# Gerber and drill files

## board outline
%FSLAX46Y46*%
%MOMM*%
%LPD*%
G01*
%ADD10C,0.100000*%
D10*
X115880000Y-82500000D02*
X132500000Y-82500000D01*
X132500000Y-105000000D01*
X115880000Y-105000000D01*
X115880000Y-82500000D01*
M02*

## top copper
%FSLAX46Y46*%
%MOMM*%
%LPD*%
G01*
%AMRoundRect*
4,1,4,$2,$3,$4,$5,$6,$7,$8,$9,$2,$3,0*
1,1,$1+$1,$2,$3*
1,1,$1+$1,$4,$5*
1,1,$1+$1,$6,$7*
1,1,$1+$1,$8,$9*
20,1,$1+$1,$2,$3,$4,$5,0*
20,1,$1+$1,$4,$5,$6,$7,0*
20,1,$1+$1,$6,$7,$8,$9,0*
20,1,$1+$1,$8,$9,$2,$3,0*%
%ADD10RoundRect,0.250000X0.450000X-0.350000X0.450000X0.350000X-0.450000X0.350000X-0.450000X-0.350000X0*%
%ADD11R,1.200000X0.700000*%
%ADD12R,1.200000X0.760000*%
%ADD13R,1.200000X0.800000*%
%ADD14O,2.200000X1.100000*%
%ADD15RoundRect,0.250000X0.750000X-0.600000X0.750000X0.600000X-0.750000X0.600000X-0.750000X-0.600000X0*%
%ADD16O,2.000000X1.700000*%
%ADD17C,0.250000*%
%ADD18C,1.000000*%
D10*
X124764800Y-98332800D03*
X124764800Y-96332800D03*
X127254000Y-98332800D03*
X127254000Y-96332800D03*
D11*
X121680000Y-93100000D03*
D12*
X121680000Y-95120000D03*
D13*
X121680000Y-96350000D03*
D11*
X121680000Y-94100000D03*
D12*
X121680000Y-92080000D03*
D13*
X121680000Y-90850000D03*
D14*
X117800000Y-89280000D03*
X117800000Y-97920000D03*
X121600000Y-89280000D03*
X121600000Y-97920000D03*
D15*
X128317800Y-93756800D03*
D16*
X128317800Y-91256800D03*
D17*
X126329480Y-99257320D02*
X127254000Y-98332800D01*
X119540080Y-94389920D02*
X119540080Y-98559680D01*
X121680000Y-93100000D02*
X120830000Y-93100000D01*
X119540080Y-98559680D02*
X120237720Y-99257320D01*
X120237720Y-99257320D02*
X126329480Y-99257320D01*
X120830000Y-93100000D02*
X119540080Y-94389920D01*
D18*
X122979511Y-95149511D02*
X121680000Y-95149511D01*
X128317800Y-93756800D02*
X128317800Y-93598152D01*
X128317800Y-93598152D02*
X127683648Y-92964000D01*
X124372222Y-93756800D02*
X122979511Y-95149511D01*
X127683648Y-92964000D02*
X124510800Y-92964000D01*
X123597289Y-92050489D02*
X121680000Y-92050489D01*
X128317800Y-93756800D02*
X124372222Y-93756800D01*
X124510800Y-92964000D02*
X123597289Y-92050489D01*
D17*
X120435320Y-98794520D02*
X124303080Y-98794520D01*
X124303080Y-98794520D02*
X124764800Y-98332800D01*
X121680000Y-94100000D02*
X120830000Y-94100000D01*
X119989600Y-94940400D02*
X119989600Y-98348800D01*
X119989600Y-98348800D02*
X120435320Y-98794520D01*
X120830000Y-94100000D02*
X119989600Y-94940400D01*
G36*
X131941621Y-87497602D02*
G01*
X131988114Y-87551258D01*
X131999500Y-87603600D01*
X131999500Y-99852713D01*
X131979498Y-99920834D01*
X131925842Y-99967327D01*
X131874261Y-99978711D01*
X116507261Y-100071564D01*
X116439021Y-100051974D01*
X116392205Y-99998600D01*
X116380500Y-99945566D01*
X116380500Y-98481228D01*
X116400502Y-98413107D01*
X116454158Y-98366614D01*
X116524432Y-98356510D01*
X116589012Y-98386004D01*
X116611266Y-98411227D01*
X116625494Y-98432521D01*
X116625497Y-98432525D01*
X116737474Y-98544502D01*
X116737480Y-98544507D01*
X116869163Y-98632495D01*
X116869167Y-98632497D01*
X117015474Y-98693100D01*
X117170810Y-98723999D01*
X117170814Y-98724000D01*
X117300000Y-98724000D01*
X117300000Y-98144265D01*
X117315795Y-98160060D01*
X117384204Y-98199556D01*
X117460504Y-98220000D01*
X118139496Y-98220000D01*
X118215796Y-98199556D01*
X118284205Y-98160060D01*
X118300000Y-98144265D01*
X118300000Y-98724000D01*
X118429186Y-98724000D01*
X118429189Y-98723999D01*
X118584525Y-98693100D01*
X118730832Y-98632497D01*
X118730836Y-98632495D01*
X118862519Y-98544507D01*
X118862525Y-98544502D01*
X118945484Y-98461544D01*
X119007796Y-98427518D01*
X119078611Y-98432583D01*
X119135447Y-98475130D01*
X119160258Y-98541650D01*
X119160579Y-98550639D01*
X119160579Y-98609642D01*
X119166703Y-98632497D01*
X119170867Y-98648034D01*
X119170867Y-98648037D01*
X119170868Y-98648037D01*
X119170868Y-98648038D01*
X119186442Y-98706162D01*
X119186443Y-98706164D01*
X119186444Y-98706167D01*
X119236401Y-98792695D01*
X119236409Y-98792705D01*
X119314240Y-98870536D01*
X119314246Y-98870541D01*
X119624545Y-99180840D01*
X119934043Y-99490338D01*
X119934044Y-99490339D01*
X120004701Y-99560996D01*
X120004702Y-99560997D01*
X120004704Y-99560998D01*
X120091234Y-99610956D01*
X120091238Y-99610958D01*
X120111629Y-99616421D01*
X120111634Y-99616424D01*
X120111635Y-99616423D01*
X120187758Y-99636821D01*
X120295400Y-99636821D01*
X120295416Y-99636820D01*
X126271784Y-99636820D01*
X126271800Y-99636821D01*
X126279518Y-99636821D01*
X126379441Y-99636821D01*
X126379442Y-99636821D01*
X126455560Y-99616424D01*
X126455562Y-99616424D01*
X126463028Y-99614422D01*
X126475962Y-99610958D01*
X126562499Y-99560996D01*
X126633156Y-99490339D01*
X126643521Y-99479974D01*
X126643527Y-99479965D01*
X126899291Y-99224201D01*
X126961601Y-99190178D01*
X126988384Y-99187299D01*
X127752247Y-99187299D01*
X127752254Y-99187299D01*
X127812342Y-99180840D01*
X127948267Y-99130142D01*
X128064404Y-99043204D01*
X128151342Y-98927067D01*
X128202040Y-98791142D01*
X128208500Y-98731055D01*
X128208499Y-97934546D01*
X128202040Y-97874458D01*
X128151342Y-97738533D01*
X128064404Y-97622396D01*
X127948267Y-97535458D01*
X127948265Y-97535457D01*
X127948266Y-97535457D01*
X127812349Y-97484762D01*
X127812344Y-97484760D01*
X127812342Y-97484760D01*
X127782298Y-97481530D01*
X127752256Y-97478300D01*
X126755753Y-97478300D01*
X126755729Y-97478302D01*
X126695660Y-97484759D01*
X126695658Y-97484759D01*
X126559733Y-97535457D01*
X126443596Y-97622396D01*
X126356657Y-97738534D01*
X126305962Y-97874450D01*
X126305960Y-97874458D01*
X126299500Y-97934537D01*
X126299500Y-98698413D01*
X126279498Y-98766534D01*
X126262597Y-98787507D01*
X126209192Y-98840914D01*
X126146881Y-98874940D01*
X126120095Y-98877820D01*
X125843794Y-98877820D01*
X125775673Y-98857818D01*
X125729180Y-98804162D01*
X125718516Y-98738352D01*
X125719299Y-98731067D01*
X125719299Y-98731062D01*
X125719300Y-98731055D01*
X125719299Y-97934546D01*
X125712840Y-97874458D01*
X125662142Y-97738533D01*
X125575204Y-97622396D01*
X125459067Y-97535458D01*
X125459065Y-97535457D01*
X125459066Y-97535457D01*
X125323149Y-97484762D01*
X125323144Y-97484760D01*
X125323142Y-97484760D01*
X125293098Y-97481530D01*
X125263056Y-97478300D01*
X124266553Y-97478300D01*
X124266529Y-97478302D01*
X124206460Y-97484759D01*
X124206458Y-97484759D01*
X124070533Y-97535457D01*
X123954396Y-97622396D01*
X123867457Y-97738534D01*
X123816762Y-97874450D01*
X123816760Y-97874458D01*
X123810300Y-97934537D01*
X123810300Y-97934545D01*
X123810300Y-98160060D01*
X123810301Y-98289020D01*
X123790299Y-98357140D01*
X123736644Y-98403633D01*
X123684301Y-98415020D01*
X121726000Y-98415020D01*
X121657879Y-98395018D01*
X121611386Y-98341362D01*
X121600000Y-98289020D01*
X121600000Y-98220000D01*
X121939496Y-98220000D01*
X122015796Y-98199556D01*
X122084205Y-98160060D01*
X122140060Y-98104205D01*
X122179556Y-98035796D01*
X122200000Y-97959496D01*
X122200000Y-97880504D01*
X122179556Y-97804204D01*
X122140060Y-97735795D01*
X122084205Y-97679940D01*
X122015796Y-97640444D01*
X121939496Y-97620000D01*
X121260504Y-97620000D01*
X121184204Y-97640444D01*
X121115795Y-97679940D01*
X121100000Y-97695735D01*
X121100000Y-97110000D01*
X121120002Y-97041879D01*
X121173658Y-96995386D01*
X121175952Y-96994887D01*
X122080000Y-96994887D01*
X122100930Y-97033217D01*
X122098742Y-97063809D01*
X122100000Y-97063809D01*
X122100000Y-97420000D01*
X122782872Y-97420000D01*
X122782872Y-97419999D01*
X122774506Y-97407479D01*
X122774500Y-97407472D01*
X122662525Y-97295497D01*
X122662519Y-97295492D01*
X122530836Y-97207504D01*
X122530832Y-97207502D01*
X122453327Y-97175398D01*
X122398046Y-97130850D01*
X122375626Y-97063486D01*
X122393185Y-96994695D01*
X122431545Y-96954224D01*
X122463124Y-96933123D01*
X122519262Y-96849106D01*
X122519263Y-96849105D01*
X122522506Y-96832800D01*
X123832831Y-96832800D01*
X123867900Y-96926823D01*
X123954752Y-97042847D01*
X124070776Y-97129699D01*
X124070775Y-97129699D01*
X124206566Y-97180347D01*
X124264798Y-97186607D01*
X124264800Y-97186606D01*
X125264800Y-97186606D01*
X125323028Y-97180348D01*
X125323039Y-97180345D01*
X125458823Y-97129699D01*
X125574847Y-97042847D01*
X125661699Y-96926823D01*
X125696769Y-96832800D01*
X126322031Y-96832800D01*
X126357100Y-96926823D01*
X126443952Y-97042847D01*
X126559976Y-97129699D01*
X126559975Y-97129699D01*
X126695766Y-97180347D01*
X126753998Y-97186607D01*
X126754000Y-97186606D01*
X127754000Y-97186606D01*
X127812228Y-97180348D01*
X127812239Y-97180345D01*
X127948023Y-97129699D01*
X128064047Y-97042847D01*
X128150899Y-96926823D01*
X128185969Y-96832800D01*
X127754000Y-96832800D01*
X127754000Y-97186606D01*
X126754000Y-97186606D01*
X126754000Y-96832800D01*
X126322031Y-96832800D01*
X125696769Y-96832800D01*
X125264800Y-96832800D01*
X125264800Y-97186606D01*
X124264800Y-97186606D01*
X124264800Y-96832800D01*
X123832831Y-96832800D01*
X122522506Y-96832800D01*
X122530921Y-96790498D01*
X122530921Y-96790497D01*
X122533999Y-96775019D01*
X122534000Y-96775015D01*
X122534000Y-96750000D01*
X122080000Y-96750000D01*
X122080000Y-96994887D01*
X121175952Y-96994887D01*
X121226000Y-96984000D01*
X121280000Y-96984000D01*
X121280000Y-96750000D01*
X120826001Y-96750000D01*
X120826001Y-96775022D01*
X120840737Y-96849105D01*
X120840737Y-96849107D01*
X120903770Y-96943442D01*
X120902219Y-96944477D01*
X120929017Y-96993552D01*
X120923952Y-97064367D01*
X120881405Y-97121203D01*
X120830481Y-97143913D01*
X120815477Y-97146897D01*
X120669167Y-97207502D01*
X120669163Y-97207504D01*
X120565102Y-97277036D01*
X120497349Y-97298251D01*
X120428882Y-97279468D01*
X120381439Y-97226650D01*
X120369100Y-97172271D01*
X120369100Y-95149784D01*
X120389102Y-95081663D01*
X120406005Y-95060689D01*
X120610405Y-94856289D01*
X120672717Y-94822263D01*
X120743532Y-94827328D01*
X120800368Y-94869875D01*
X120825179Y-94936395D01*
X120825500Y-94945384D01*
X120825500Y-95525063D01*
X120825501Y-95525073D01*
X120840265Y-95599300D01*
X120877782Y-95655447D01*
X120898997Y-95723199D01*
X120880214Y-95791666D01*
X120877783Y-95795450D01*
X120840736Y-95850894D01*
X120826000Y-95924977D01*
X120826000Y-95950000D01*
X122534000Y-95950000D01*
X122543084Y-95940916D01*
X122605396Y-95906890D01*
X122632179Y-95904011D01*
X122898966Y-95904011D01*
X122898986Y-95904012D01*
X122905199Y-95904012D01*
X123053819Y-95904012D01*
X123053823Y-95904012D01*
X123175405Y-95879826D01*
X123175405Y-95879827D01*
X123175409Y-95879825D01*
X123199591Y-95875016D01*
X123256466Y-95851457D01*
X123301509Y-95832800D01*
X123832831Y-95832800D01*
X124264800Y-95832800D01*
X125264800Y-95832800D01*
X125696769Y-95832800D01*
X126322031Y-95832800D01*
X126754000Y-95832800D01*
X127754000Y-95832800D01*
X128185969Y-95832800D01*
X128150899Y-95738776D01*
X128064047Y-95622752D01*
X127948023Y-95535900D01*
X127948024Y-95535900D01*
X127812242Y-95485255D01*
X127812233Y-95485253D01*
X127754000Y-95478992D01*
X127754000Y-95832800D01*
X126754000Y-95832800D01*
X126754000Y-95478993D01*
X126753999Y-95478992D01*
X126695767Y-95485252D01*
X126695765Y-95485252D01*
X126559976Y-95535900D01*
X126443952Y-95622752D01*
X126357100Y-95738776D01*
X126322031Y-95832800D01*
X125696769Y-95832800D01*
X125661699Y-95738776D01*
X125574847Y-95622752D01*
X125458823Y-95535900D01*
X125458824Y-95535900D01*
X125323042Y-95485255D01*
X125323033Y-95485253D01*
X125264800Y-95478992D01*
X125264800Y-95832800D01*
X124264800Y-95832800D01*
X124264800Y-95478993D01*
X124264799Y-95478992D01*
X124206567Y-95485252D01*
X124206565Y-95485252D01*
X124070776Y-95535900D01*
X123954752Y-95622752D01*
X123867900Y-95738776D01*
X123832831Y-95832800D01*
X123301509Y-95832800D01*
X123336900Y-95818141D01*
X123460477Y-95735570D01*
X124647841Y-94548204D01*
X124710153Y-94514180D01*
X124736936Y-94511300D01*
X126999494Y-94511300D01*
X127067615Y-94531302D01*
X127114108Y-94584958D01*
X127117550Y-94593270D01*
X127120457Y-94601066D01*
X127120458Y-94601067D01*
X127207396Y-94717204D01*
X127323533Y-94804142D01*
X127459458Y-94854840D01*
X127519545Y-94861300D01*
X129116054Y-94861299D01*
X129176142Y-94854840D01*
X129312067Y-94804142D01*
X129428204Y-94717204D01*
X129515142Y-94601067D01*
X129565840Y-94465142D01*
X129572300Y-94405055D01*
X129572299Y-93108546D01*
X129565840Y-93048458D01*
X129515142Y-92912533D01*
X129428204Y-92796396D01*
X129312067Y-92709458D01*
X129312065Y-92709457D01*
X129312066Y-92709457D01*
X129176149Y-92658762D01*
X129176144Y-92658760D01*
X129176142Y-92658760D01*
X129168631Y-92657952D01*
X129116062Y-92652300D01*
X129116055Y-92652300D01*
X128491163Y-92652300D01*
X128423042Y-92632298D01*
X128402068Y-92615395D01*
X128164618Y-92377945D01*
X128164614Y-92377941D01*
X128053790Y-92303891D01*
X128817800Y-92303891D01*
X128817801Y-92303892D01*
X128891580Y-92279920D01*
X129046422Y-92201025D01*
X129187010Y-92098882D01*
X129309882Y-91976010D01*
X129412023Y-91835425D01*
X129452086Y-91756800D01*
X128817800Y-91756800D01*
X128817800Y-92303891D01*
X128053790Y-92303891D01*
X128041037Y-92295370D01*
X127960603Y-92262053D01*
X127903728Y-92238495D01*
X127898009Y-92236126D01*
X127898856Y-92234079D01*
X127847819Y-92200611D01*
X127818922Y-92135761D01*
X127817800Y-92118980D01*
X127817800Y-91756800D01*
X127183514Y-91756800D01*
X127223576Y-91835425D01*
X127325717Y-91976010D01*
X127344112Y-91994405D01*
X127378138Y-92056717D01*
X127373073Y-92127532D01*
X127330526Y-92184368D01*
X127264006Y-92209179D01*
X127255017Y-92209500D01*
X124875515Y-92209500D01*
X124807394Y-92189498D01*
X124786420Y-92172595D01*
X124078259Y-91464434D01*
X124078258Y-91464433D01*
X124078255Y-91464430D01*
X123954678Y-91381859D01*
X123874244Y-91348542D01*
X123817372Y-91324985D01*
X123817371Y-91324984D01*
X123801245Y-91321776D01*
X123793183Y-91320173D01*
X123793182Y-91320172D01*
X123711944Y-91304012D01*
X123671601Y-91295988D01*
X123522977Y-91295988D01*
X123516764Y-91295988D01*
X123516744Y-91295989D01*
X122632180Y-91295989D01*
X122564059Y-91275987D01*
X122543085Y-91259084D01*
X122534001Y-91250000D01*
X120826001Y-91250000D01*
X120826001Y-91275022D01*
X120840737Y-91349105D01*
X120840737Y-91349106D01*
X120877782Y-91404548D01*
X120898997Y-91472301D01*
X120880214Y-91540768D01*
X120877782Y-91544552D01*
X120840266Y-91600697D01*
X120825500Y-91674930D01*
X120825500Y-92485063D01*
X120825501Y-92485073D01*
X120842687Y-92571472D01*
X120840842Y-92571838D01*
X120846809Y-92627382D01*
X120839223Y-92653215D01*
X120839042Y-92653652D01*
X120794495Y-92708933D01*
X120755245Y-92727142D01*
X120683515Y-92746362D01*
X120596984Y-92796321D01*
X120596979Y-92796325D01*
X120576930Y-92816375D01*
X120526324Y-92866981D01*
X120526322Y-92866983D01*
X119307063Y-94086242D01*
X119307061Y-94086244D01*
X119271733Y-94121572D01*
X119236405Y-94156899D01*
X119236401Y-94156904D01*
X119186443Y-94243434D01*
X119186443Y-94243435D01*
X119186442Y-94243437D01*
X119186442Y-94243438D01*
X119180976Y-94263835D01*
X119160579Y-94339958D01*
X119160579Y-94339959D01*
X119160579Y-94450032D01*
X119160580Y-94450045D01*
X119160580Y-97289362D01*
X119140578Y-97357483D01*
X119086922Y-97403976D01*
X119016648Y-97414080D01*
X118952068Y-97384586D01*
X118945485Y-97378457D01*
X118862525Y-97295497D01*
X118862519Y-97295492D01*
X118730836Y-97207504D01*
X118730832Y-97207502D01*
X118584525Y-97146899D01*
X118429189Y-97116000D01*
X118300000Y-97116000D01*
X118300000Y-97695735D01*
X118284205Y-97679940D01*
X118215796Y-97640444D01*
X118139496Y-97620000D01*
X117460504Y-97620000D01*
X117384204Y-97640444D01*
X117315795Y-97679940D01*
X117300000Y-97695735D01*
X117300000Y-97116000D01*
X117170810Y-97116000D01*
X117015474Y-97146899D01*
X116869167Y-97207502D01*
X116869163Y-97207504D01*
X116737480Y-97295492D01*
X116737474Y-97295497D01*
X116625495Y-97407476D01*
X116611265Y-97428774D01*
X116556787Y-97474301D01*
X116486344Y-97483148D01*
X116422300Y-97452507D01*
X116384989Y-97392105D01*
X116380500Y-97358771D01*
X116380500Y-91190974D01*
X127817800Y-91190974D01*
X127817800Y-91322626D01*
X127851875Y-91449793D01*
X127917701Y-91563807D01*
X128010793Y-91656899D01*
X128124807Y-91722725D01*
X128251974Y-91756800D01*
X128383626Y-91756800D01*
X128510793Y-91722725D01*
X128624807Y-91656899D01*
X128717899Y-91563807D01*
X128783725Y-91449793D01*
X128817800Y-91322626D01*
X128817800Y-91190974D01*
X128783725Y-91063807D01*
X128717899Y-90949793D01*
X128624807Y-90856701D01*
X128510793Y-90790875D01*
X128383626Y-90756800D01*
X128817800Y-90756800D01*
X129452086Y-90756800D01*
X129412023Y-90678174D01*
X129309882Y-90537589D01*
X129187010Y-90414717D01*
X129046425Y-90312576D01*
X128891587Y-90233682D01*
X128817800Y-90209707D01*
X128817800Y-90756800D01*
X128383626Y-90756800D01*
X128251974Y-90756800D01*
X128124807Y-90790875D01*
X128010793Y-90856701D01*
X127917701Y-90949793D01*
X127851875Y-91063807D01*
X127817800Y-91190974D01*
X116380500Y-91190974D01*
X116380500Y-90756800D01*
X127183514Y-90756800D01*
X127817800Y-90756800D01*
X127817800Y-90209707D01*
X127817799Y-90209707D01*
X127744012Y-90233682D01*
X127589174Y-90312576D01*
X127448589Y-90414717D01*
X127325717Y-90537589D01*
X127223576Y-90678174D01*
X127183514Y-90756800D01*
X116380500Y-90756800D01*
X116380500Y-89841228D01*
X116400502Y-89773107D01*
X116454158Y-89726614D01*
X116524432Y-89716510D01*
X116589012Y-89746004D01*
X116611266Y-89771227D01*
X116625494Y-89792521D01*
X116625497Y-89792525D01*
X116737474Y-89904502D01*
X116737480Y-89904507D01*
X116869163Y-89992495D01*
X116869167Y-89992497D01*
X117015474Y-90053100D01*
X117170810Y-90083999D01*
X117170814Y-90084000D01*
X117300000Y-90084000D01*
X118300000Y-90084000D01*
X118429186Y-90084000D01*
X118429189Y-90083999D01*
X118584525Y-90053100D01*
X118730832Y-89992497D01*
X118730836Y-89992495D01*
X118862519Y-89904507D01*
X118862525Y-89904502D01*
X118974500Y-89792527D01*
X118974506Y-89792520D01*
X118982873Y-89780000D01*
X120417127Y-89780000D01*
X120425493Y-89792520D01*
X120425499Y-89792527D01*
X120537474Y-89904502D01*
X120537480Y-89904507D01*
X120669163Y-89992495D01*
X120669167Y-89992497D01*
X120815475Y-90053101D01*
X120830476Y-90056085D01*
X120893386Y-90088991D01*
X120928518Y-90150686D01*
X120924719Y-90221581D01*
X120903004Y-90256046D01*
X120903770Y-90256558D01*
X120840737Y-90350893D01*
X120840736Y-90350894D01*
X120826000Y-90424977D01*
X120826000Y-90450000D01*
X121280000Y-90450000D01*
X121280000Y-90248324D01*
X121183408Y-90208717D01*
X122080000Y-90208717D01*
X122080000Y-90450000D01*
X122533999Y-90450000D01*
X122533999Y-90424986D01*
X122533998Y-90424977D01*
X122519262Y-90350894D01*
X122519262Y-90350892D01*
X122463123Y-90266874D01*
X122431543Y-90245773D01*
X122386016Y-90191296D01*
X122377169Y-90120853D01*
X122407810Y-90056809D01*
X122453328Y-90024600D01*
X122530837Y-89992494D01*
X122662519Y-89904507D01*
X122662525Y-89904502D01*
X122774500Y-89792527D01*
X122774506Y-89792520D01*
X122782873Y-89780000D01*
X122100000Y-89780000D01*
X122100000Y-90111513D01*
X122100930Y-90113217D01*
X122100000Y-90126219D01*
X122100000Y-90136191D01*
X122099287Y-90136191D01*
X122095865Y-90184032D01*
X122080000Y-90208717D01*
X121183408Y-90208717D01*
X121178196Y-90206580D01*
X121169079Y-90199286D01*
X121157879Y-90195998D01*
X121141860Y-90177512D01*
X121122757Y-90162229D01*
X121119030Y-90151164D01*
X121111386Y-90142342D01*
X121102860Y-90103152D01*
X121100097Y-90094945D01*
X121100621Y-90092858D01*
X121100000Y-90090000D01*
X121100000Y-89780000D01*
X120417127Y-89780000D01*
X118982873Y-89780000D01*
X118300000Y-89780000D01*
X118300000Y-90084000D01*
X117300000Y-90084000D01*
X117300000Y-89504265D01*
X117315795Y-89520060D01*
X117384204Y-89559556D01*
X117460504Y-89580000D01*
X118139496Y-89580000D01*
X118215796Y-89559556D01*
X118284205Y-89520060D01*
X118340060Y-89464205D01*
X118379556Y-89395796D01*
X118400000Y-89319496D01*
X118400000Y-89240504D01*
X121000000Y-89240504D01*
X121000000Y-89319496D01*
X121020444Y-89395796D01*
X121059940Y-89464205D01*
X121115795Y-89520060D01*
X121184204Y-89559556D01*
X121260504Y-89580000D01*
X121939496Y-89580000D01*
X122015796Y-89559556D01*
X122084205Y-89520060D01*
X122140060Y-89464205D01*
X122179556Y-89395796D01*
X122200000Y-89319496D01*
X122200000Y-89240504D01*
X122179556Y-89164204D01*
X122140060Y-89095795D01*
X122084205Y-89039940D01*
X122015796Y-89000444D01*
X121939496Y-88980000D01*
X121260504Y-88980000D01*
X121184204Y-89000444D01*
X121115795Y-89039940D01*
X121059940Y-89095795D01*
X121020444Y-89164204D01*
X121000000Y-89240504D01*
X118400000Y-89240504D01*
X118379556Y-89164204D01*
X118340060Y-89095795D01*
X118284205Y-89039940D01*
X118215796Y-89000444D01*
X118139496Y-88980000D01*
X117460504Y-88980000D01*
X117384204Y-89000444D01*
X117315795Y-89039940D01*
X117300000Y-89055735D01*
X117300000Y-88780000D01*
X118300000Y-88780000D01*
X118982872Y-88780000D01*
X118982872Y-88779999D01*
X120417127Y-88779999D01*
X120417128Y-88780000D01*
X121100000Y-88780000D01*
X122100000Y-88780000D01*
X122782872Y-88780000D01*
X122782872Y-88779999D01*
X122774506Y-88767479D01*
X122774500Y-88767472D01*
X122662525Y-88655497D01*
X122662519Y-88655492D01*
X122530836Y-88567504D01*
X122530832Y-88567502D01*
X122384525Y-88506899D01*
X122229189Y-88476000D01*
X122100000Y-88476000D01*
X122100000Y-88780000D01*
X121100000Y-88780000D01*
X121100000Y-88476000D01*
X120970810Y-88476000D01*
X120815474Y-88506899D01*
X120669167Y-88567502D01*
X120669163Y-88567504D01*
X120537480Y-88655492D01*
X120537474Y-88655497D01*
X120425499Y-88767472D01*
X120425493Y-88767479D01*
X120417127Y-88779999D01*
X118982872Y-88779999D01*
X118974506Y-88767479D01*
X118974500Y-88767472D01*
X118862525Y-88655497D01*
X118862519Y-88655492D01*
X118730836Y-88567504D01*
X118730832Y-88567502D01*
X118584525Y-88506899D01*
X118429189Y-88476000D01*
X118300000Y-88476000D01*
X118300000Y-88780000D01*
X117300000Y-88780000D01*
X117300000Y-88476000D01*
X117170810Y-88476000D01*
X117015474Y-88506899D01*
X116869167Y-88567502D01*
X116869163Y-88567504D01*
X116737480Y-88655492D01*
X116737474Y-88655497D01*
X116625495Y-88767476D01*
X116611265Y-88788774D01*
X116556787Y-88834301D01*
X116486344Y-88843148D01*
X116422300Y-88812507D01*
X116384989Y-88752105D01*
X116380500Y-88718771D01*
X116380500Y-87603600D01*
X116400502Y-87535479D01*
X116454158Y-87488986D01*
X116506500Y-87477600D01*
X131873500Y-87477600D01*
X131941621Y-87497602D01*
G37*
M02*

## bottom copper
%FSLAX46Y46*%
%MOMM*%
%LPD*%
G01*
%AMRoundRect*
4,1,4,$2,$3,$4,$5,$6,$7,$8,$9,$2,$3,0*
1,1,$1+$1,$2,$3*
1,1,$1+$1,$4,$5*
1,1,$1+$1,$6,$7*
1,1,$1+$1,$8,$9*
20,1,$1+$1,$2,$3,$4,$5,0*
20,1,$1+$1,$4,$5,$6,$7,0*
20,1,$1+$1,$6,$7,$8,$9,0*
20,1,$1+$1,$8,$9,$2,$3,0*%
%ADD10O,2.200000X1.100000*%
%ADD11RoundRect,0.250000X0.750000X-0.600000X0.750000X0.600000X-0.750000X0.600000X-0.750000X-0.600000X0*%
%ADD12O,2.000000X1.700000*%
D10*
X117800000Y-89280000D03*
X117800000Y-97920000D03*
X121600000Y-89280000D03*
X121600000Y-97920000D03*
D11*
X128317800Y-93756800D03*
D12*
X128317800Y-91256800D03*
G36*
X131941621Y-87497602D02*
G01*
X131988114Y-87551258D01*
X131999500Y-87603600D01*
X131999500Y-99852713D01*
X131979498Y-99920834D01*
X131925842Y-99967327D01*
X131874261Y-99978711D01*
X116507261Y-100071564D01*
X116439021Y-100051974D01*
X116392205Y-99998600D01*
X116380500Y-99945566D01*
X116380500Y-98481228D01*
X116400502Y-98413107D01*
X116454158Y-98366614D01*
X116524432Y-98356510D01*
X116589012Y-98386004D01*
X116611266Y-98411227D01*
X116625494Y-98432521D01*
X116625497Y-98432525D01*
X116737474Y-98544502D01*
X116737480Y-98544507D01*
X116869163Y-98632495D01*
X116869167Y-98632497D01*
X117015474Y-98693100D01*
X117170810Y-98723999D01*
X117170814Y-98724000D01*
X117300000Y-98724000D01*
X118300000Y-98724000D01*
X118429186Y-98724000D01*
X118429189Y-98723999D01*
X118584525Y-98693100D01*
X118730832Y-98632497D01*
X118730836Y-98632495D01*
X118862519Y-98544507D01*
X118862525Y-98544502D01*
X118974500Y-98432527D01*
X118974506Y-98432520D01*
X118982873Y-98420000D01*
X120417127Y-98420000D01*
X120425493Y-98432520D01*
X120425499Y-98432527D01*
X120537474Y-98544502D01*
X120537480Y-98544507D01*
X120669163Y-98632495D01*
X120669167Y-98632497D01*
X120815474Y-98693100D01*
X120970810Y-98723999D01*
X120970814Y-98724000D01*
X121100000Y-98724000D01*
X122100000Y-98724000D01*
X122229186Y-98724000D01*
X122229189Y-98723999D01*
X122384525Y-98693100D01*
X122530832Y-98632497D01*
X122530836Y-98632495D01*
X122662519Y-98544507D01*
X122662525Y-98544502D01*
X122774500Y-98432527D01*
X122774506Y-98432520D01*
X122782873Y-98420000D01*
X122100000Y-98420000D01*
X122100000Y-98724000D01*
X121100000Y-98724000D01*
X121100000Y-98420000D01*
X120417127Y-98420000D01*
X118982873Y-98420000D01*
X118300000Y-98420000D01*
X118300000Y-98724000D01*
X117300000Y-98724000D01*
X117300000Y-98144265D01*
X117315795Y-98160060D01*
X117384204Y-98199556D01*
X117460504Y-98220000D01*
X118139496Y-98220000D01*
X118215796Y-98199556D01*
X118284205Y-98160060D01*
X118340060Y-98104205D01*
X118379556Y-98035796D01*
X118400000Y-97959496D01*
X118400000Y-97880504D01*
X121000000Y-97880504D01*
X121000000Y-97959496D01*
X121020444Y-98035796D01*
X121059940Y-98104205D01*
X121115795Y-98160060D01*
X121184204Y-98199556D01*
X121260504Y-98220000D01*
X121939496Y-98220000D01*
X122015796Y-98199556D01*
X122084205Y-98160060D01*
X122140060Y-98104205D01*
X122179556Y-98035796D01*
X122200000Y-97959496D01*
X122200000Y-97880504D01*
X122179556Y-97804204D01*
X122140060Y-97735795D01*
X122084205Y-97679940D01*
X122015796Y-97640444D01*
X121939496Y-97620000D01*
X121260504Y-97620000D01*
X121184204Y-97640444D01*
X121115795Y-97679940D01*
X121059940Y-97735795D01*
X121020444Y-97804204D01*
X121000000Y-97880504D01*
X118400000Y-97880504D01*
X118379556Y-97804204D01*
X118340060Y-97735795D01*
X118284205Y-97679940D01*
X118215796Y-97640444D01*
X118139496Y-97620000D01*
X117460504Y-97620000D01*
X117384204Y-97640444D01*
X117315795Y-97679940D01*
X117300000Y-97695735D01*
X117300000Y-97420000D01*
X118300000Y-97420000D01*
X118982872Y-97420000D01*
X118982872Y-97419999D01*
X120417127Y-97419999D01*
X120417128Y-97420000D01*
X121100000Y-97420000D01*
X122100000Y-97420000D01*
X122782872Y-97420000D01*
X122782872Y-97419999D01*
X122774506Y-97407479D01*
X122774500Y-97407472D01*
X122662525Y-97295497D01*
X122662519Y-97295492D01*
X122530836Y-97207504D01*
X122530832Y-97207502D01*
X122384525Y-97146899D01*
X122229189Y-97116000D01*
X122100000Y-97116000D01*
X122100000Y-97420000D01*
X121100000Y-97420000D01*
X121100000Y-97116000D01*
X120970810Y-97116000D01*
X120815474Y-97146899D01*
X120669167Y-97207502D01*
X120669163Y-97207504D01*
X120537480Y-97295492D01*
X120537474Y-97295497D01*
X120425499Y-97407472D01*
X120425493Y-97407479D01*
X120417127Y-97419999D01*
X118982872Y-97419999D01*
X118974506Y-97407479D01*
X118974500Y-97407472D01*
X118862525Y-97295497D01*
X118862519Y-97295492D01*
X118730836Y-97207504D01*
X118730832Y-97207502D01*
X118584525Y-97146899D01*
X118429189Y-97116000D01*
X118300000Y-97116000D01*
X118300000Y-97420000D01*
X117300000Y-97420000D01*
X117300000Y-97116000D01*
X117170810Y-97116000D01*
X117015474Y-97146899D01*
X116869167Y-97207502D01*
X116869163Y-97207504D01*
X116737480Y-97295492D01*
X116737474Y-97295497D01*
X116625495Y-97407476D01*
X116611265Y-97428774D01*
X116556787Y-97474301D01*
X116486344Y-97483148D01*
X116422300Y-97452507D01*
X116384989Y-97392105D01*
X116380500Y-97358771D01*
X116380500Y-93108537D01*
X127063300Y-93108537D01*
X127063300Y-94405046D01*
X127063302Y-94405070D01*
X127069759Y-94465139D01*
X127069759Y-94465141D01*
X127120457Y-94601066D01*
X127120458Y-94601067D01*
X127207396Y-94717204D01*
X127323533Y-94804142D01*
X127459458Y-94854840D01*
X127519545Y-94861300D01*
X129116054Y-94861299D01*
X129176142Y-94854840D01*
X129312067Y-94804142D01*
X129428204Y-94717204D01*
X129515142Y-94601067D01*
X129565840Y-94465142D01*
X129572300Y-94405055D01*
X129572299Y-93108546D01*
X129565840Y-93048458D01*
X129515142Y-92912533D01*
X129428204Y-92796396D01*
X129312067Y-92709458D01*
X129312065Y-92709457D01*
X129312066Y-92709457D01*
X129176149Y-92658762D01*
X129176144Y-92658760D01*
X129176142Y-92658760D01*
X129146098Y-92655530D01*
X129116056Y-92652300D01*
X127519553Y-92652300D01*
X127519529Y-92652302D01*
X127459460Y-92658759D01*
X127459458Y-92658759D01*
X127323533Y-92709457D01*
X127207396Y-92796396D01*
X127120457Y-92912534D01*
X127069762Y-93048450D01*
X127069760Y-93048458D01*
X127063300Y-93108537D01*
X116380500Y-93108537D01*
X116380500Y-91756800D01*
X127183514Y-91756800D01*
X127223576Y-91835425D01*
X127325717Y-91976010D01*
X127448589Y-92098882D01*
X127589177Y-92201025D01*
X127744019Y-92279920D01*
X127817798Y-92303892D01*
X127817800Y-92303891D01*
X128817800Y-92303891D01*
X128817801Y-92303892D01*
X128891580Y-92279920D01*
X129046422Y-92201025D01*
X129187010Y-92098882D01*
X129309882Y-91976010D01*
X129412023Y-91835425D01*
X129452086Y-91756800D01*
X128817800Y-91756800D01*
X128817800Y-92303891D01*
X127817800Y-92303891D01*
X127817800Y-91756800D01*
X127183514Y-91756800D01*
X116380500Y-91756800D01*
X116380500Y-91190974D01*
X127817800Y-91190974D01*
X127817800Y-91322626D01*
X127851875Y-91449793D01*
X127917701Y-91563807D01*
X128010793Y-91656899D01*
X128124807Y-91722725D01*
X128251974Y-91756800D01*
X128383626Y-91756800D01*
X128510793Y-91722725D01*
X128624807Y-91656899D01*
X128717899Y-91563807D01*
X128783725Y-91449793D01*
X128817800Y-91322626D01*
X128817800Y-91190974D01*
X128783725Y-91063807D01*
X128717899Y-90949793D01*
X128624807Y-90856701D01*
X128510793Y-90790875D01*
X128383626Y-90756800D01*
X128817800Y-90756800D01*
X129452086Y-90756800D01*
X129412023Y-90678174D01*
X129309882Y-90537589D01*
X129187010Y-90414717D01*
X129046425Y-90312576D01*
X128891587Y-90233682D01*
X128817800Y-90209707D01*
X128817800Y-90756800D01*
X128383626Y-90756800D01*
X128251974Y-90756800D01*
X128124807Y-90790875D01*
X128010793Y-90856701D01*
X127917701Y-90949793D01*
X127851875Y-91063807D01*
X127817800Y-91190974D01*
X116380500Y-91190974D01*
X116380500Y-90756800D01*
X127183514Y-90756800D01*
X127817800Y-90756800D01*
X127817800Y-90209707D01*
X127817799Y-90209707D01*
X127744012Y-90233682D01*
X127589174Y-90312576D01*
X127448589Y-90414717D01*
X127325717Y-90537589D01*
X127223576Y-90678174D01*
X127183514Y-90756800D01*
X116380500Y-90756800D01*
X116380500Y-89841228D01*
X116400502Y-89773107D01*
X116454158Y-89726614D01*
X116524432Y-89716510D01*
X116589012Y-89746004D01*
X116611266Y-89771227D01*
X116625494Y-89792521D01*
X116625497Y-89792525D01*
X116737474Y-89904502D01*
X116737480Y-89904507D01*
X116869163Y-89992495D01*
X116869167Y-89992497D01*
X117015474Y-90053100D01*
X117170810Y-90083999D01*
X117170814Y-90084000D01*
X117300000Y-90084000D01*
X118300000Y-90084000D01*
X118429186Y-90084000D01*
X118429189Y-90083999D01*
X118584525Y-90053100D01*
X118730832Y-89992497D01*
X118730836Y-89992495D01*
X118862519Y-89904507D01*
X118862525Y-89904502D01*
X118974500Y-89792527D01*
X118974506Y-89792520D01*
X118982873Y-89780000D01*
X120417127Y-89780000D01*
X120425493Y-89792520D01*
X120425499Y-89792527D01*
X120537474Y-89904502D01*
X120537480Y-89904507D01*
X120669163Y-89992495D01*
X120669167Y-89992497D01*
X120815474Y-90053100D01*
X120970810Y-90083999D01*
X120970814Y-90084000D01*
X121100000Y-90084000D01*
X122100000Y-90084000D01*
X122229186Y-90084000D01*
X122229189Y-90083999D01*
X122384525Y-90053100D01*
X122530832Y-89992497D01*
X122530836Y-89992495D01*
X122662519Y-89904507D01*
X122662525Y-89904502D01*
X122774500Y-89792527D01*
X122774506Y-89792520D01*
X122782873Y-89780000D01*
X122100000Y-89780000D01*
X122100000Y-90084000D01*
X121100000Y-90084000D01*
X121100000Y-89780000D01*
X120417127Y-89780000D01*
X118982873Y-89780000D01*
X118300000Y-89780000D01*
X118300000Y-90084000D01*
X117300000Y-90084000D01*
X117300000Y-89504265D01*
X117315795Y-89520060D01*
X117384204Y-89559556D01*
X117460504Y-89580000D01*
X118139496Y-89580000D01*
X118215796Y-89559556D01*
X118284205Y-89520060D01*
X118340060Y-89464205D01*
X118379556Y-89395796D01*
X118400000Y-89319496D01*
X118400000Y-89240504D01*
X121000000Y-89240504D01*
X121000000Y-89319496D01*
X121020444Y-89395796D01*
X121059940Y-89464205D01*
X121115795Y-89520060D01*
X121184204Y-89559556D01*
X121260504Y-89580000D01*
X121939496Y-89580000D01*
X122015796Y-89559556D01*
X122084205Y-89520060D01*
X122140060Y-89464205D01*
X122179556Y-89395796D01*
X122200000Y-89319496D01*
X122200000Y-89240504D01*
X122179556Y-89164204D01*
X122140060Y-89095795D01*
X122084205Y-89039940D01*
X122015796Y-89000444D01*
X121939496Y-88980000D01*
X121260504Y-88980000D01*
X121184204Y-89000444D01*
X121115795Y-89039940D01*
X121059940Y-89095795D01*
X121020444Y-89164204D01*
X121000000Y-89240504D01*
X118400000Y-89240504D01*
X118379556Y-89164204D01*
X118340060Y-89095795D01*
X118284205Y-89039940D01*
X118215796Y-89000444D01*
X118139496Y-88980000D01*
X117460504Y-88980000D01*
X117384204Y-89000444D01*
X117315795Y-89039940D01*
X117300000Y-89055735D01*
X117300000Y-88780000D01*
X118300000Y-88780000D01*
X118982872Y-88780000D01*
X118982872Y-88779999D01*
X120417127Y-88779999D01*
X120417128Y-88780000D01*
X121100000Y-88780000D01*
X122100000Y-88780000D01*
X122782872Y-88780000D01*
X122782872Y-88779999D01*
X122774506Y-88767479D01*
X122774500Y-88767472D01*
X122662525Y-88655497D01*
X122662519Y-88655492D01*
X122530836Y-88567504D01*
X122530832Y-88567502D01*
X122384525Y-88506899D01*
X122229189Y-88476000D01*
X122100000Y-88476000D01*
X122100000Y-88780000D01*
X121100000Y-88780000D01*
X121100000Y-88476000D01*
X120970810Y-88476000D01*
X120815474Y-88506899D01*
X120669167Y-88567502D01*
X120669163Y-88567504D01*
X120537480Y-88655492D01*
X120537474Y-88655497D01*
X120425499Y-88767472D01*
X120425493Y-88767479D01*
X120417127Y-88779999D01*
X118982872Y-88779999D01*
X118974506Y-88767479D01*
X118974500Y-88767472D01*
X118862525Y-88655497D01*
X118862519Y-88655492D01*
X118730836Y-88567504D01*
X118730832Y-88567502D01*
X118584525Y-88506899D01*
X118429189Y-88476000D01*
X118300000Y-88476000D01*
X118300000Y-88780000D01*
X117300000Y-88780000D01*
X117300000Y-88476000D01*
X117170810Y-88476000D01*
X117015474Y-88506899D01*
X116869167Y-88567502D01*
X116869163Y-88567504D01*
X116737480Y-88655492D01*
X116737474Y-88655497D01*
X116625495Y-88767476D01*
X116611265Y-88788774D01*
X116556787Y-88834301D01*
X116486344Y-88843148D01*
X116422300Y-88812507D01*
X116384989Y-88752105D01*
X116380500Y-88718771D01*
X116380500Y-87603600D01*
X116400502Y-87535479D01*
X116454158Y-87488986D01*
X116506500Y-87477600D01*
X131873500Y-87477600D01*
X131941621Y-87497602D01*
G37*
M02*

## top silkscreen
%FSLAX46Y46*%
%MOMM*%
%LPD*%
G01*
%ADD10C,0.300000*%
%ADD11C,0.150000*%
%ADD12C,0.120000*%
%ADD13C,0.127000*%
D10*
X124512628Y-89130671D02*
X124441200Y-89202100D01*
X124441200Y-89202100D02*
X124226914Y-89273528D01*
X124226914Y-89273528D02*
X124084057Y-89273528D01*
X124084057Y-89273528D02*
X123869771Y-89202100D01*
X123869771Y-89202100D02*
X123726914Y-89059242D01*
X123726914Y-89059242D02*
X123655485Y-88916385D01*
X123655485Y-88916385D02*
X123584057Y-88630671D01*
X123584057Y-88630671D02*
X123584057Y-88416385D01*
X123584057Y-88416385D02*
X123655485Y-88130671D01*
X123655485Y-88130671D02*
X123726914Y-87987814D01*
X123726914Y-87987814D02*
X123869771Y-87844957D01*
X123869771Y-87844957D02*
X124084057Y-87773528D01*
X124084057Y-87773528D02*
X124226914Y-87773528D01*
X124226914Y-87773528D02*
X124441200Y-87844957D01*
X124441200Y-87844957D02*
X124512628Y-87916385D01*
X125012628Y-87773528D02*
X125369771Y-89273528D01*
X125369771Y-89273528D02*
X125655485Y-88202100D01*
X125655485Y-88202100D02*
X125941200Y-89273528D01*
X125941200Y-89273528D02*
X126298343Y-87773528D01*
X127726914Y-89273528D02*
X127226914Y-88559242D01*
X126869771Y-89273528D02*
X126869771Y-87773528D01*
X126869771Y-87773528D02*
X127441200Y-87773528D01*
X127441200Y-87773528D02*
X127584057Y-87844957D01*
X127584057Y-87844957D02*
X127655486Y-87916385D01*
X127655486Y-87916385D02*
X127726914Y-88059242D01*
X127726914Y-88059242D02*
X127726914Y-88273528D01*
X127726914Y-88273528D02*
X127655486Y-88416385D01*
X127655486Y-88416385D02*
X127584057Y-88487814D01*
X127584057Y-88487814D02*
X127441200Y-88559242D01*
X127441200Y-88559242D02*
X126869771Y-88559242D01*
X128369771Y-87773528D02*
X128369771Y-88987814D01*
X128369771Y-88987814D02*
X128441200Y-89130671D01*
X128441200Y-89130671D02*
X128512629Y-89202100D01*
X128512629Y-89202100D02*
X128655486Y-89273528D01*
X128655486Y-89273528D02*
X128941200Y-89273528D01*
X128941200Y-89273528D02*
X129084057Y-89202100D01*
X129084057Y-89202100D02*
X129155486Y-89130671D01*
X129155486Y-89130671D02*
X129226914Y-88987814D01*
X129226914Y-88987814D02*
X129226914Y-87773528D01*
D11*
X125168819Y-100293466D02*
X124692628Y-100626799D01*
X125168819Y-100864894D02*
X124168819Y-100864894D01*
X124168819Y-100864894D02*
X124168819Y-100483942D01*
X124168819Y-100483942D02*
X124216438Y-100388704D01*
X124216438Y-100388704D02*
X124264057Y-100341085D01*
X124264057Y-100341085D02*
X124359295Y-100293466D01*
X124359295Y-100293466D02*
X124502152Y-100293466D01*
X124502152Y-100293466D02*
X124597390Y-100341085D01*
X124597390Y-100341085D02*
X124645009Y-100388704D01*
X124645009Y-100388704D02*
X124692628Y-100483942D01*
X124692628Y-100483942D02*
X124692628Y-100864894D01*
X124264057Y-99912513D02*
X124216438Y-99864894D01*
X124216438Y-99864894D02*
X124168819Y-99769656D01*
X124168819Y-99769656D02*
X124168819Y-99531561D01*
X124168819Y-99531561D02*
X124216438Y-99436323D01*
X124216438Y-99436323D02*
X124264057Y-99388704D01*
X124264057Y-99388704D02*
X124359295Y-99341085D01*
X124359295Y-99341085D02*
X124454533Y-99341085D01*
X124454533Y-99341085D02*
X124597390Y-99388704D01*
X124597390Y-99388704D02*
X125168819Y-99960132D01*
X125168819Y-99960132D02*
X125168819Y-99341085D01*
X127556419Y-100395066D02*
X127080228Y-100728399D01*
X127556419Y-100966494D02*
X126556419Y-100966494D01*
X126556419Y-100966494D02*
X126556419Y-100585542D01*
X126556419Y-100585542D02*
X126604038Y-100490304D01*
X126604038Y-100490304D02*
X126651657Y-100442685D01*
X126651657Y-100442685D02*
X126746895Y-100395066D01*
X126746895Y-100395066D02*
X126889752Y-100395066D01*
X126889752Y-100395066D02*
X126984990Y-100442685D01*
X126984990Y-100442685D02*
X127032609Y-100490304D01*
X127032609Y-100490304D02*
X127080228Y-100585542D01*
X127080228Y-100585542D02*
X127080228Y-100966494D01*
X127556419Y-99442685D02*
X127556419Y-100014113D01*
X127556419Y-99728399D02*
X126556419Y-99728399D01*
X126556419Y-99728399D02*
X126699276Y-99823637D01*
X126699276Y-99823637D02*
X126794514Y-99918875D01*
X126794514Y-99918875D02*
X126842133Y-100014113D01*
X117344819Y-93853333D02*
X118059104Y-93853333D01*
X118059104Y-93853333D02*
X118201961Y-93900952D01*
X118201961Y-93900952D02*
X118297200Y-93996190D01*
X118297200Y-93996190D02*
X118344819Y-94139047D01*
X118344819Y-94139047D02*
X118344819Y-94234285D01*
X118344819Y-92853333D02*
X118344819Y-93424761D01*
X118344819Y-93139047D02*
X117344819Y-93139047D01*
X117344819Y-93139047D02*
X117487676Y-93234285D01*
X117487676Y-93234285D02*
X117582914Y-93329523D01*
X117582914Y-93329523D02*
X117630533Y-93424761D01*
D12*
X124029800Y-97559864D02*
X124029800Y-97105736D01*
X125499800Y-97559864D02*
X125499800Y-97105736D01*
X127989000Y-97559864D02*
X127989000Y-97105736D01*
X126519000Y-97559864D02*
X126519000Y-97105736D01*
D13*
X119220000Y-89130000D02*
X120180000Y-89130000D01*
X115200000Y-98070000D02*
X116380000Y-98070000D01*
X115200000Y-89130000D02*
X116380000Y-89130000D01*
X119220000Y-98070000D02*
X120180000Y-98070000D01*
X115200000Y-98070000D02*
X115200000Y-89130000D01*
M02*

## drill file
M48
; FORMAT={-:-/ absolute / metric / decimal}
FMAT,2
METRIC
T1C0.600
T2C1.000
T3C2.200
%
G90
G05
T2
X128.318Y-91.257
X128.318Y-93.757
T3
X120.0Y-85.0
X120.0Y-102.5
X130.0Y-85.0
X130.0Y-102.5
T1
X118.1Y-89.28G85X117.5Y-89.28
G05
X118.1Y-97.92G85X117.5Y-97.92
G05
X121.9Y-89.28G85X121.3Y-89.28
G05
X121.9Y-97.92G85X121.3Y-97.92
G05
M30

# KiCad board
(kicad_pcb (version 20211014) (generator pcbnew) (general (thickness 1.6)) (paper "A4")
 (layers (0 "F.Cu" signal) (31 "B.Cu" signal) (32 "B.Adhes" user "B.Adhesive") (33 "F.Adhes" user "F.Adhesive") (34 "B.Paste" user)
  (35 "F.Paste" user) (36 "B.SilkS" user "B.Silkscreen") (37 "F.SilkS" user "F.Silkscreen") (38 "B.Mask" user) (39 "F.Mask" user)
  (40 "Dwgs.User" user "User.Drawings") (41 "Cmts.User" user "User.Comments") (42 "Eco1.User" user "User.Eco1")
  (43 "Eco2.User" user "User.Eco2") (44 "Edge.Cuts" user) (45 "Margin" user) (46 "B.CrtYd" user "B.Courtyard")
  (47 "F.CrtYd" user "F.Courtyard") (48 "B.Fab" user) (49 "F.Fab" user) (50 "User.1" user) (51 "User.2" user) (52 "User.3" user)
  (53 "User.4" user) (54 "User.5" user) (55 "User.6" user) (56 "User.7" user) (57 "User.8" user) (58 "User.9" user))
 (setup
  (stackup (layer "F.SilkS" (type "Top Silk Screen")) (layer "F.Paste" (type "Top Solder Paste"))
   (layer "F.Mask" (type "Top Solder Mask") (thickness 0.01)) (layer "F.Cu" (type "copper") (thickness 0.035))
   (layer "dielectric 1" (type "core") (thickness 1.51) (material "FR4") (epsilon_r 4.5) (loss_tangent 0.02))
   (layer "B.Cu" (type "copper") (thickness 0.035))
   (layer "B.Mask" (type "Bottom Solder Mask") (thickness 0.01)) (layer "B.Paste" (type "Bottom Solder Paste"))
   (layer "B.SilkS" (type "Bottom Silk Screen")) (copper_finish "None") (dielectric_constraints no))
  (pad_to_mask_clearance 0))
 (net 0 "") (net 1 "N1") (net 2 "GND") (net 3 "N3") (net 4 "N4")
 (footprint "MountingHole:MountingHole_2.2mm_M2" (layer "F.Cu") (at 130 102.5)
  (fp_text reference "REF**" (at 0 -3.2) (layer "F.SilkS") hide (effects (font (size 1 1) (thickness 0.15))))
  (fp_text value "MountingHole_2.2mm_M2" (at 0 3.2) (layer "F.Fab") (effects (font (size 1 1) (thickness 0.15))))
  (pad "" np_thru_hole circle locked (at 0 0) (size 2.2 2.2) (drill 2.2) (layers *.Cu *.Mask)))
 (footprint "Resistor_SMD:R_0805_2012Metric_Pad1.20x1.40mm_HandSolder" (layer "F.Cu") (at 124.7648 97.3328 90)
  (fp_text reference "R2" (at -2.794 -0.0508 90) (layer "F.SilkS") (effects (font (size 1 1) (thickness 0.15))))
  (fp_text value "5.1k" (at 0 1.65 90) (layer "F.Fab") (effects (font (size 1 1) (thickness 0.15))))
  (fp_line (start -0.227064 -0.735) (end 0.227064 -0.735) (layer "F.SilkS") (width 0.12))
  (fp_line (start -0.227064 0.735) (end 0.227064 0.735) (layer "F.SilkS") (width 0.12))
  (pad "1" smd roundrect locked (at -1 0 90) (size 1.2 1.4) (layers "F.Cu" "F.Paste" "F.Mask") (roundrect_rratio 0.2083333333) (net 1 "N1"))
  (pad "2" smd roundrect locked (at 1 0 90) (size 1.2 1.4) (layers "F.Cu" "F.Paste" "F.Mask") (roundrect_rratio 0.2083333333) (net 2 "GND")))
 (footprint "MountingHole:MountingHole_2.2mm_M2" (layer "F.Cu") (at 120 102.5)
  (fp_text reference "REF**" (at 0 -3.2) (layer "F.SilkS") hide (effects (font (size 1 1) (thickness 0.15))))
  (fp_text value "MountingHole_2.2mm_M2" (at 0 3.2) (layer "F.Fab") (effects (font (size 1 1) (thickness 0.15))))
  (pad "" np_thru_hole circle locked (at 0 0) (size 2.2 2.2) (drill 2.2) (layers *.Cu *.Mask)))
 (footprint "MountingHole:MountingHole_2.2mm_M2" (layer "F.Cu") (at 120 85)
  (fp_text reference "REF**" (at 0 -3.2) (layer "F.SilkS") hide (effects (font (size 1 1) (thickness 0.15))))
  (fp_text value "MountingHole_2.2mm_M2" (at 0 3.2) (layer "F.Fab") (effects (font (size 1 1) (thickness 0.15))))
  (pad "" np_thru_hole circle locked (at 0 0) (size 2.2 2.2) (drill 2.2) (layers *.Cu *.Mask)))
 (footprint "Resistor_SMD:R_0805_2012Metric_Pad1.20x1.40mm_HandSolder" (layer "F.Cu") (at 127.254 97.3328 90)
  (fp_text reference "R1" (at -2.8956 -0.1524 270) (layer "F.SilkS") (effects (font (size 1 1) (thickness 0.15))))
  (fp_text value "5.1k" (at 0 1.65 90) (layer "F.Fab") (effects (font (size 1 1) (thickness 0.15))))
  (fp_line (start -0.227064 0.735) (end 0.227064 0.735) (layer "F.SilkS") (width 0.12))
  (fp_line (start -0.227064 -0.735) (end 0.227064 -0.735) (layer "F.SilkS") (width 0.12))
  (pad "1" smd roundrect locked (at -1 0 90) (size 1.2 1.4) (layers "F.Cu" "F.Paste" "F.Mask") (roundrect_rratio 0.2083333333) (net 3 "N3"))
  (pad "2" smd roundrect locked (at 1 0 90) (size 1.2 1.4) (layers "F.Cu" "F.Paste" "F.Mask") (roundrect_rratio 0.2083333333) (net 2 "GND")))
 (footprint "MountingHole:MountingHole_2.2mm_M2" (layer "F.Cu") (at 130 85)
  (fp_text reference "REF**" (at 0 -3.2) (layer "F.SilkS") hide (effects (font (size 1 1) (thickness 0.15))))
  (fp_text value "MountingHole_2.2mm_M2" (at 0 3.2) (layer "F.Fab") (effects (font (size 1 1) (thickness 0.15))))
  (pad "" np_thru_hole circle locked (at 0 0) (size 2.2 2.2) (drill 2.2) (layers *.Cu *.Mask)))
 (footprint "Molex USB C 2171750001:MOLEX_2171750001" (layer "F.Cu") (at 117.8 93.6 -90)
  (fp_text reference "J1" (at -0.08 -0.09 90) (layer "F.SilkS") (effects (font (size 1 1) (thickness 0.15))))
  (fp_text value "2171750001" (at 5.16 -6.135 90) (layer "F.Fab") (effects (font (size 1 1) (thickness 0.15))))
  (fp_line (start -4.47 -1.42) (end -4.47 -2.38) (layer "F.SilkS") (width 0.127))
  (fp_line (start 4.47 2.6) (end 4.47 1.42) (layer "F.SilkS") (width 0.127))
  (fp_line (start -4.47 2.6) (end -4.47 1.42) (layer "F.SilkS") (width 0.127))
  (fp_line (start 4.47 -1.42) (end 4.47 -2.38) (layer "F.SilkS") (width 0.127))
  (fp_line (start 4.47 2.6) (end -4.47 2.6) (layer "F.SilkS") (width 0.127))
  (pad "A5" smd rect (at -0.5 -3.88 270) (size 0.7 1.2) (layers "F.Cu" "F.Paste" "F.Mask") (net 3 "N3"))
  (pad "A9" smd rect (at 1.52 -3.88 270) (size 0.76 1.2) (layers "F.Cu" "F.Paste" "F.Mask") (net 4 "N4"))
  (pad "A12" smd rect (at 2.75 -3.88 270) (size 0.8 1.2) (layers "F.Cu" "F.Paste" "F.Mask") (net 2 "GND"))
  (pad "B5" smd rect (at 0.5 -3.88 270) (size 0.7 1.2) (layers "F.Cu" "F.Paste" "F.Mask") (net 1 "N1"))
  (pad "B9" smd rect (at -1.52 -3.88 270) (size 0.76 1.2) (layers "F.Cu" "F.Paste" "F.Mask") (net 4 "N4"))
  (pad "B12" smd rect (at -2.75 -3.88 270) (size 0.8 1.2) (layers "F.Cu" "F.Paste" "F.Mask") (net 2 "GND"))
  (pad "S1" thru_hole oval (at -4.32 0 270) (size 1.1 2.2) (drill oval 0.6 1.2) (layers *.Cu *.Mask) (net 2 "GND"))
  (pad "S2" thru_hole oval (at 4.32 0 270) (size 1.1 2.2) (drill oval 0.6 1.2) (layers *.Cu *.Mask) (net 2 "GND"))
  (pad "S3" thru_hole oval (at -4.32 -3.8 270) (size 1.1 2.2) (drill oval 0.6 1.2) (layers *.Cu *.Mask) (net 2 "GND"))
  (pad "S4" thru_hole oval (at 4.32 -3.8 270) (size 1.1 2.2) (drill oval 0.6 1.2) (layers *.Cu *.Mask) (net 2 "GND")))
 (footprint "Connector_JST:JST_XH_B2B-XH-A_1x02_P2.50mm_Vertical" (layer "B.Cu") (at 128.3178 93.7568 90)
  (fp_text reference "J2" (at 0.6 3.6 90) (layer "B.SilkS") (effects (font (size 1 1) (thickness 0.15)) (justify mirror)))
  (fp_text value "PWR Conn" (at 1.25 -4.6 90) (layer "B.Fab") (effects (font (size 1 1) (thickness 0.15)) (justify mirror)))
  (pad "1" thru_hole roundrect locked (at 0 0 90) (size 1.7 2) (drill 1) (layers *.Cu *.Mask) (roundrect_rratio 0.1470588235) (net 4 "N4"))
  (pad "2" thru_hole oval locked (at 2.5 0 90) (size 1.7 2) (drill 1) (layers *.Cu *.Mask) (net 2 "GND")))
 (gr_rect (start 115.88 82.5) (end 132.5 105) (layer "Edge.Cuts") (width 0.1) (fill none))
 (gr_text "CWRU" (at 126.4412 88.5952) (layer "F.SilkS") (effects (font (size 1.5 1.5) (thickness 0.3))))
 (segment (start 126.32948 99.25732) (end 127.254 98.3328) (width 0.25) (layer "F.Cu") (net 3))
 (segment (start 119.54008 94.38992) (end 119.54008 98.55968) (width 0.25) (layer "F.Cu") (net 3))
 (segment (start 121.68 93.1) (end 120.83 93.1) (width 0.25) (layer "F.Cu") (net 3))
 (segment (start 119.54008 98.55968) (end 120.23772 99.25732) (width 0.25) (layer "F.Cu") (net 3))
 (segment (start 120.23772 99.25732) (end 126.32948 99.25732) (width 0.25) (layer "F.Cu") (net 3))
 (segment (start 120.83 93.1) (end 119.54008 94.38992) (width 0.25) (layer "F.Cu") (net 3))
 (segment (start 122.979511 95.149511) (end 121.68 95.149511) (width 1) (layer "F.Cu") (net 4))
 (segment (start 128.3178 93.7568) (end 128.3178 93.598152) (width 1) (layer "F.Cu") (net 4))
 (segment (start 128.3178 93.598152) (end 127.683648 92.964) (width 1) (layer "F.Cu") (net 4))
 (segment (start 124.372222 93.7568) (end 122.979511 95.149511) (width 1) (layer "F.Cu") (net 4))
 (segment (start 127.683648 92.964) (end 124.5108 92.964) (width 1) (layer "F.Cu") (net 4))
 (segment (start 123.597289 92.050489) (end 121.68 92.050489) (width 1) (layer "F.Cu") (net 4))
 (segment (start 128.3178 93.7568) (end 124.372222 93.7568) (width 1) (layer "F.Cu") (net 4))
 (segment (start 124.5108 92.964) (end 123.597289 92.050489) (width 1) (layer "F.Cu") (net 4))
 (segment (start 120.43532 98.79452) (end 124.30308 98.79452) (width 0.25) (layer "F.Cu") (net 1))
 (segment (start 124.30308 98.79452) (end 124.7648 98.3328) (width 0.25) (layer "F.Cu") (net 1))
 (segment (start 121.68 94.1) (end 120.83 94.1) (width 0.25) (layer "F.Cu") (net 1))
 (segment (start 119.9896 94.9404) (end 119.9896 98.3488) (width 0.25) (layer "F.Cu") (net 1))
 (segment (start 119.9896 98.3488) (end 120.43532 98.79452) (width 0.25) (layer "F.Cu") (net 1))
 (segment (start 120.83 94.1) (end 119.9896 94.9404) (width 0.25) (layer "F.Cu") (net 1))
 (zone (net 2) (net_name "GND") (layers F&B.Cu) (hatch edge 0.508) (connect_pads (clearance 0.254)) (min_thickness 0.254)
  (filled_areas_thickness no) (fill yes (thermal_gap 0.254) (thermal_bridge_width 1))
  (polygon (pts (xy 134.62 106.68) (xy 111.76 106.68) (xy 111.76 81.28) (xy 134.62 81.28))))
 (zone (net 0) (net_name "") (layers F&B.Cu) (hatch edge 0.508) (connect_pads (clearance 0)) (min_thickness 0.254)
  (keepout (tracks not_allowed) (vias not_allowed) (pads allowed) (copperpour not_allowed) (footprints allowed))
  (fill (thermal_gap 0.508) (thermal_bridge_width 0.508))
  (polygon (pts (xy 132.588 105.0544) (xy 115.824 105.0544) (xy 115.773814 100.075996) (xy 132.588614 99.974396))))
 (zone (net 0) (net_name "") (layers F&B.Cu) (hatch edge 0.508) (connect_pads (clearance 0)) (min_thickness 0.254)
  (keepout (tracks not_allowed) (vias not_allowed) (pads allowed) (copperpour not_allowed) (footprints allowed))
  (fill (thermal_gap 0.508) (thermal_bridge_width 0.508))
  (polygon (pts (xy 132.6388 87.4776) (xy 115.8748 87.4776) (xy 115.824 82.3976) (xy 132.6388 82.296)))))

